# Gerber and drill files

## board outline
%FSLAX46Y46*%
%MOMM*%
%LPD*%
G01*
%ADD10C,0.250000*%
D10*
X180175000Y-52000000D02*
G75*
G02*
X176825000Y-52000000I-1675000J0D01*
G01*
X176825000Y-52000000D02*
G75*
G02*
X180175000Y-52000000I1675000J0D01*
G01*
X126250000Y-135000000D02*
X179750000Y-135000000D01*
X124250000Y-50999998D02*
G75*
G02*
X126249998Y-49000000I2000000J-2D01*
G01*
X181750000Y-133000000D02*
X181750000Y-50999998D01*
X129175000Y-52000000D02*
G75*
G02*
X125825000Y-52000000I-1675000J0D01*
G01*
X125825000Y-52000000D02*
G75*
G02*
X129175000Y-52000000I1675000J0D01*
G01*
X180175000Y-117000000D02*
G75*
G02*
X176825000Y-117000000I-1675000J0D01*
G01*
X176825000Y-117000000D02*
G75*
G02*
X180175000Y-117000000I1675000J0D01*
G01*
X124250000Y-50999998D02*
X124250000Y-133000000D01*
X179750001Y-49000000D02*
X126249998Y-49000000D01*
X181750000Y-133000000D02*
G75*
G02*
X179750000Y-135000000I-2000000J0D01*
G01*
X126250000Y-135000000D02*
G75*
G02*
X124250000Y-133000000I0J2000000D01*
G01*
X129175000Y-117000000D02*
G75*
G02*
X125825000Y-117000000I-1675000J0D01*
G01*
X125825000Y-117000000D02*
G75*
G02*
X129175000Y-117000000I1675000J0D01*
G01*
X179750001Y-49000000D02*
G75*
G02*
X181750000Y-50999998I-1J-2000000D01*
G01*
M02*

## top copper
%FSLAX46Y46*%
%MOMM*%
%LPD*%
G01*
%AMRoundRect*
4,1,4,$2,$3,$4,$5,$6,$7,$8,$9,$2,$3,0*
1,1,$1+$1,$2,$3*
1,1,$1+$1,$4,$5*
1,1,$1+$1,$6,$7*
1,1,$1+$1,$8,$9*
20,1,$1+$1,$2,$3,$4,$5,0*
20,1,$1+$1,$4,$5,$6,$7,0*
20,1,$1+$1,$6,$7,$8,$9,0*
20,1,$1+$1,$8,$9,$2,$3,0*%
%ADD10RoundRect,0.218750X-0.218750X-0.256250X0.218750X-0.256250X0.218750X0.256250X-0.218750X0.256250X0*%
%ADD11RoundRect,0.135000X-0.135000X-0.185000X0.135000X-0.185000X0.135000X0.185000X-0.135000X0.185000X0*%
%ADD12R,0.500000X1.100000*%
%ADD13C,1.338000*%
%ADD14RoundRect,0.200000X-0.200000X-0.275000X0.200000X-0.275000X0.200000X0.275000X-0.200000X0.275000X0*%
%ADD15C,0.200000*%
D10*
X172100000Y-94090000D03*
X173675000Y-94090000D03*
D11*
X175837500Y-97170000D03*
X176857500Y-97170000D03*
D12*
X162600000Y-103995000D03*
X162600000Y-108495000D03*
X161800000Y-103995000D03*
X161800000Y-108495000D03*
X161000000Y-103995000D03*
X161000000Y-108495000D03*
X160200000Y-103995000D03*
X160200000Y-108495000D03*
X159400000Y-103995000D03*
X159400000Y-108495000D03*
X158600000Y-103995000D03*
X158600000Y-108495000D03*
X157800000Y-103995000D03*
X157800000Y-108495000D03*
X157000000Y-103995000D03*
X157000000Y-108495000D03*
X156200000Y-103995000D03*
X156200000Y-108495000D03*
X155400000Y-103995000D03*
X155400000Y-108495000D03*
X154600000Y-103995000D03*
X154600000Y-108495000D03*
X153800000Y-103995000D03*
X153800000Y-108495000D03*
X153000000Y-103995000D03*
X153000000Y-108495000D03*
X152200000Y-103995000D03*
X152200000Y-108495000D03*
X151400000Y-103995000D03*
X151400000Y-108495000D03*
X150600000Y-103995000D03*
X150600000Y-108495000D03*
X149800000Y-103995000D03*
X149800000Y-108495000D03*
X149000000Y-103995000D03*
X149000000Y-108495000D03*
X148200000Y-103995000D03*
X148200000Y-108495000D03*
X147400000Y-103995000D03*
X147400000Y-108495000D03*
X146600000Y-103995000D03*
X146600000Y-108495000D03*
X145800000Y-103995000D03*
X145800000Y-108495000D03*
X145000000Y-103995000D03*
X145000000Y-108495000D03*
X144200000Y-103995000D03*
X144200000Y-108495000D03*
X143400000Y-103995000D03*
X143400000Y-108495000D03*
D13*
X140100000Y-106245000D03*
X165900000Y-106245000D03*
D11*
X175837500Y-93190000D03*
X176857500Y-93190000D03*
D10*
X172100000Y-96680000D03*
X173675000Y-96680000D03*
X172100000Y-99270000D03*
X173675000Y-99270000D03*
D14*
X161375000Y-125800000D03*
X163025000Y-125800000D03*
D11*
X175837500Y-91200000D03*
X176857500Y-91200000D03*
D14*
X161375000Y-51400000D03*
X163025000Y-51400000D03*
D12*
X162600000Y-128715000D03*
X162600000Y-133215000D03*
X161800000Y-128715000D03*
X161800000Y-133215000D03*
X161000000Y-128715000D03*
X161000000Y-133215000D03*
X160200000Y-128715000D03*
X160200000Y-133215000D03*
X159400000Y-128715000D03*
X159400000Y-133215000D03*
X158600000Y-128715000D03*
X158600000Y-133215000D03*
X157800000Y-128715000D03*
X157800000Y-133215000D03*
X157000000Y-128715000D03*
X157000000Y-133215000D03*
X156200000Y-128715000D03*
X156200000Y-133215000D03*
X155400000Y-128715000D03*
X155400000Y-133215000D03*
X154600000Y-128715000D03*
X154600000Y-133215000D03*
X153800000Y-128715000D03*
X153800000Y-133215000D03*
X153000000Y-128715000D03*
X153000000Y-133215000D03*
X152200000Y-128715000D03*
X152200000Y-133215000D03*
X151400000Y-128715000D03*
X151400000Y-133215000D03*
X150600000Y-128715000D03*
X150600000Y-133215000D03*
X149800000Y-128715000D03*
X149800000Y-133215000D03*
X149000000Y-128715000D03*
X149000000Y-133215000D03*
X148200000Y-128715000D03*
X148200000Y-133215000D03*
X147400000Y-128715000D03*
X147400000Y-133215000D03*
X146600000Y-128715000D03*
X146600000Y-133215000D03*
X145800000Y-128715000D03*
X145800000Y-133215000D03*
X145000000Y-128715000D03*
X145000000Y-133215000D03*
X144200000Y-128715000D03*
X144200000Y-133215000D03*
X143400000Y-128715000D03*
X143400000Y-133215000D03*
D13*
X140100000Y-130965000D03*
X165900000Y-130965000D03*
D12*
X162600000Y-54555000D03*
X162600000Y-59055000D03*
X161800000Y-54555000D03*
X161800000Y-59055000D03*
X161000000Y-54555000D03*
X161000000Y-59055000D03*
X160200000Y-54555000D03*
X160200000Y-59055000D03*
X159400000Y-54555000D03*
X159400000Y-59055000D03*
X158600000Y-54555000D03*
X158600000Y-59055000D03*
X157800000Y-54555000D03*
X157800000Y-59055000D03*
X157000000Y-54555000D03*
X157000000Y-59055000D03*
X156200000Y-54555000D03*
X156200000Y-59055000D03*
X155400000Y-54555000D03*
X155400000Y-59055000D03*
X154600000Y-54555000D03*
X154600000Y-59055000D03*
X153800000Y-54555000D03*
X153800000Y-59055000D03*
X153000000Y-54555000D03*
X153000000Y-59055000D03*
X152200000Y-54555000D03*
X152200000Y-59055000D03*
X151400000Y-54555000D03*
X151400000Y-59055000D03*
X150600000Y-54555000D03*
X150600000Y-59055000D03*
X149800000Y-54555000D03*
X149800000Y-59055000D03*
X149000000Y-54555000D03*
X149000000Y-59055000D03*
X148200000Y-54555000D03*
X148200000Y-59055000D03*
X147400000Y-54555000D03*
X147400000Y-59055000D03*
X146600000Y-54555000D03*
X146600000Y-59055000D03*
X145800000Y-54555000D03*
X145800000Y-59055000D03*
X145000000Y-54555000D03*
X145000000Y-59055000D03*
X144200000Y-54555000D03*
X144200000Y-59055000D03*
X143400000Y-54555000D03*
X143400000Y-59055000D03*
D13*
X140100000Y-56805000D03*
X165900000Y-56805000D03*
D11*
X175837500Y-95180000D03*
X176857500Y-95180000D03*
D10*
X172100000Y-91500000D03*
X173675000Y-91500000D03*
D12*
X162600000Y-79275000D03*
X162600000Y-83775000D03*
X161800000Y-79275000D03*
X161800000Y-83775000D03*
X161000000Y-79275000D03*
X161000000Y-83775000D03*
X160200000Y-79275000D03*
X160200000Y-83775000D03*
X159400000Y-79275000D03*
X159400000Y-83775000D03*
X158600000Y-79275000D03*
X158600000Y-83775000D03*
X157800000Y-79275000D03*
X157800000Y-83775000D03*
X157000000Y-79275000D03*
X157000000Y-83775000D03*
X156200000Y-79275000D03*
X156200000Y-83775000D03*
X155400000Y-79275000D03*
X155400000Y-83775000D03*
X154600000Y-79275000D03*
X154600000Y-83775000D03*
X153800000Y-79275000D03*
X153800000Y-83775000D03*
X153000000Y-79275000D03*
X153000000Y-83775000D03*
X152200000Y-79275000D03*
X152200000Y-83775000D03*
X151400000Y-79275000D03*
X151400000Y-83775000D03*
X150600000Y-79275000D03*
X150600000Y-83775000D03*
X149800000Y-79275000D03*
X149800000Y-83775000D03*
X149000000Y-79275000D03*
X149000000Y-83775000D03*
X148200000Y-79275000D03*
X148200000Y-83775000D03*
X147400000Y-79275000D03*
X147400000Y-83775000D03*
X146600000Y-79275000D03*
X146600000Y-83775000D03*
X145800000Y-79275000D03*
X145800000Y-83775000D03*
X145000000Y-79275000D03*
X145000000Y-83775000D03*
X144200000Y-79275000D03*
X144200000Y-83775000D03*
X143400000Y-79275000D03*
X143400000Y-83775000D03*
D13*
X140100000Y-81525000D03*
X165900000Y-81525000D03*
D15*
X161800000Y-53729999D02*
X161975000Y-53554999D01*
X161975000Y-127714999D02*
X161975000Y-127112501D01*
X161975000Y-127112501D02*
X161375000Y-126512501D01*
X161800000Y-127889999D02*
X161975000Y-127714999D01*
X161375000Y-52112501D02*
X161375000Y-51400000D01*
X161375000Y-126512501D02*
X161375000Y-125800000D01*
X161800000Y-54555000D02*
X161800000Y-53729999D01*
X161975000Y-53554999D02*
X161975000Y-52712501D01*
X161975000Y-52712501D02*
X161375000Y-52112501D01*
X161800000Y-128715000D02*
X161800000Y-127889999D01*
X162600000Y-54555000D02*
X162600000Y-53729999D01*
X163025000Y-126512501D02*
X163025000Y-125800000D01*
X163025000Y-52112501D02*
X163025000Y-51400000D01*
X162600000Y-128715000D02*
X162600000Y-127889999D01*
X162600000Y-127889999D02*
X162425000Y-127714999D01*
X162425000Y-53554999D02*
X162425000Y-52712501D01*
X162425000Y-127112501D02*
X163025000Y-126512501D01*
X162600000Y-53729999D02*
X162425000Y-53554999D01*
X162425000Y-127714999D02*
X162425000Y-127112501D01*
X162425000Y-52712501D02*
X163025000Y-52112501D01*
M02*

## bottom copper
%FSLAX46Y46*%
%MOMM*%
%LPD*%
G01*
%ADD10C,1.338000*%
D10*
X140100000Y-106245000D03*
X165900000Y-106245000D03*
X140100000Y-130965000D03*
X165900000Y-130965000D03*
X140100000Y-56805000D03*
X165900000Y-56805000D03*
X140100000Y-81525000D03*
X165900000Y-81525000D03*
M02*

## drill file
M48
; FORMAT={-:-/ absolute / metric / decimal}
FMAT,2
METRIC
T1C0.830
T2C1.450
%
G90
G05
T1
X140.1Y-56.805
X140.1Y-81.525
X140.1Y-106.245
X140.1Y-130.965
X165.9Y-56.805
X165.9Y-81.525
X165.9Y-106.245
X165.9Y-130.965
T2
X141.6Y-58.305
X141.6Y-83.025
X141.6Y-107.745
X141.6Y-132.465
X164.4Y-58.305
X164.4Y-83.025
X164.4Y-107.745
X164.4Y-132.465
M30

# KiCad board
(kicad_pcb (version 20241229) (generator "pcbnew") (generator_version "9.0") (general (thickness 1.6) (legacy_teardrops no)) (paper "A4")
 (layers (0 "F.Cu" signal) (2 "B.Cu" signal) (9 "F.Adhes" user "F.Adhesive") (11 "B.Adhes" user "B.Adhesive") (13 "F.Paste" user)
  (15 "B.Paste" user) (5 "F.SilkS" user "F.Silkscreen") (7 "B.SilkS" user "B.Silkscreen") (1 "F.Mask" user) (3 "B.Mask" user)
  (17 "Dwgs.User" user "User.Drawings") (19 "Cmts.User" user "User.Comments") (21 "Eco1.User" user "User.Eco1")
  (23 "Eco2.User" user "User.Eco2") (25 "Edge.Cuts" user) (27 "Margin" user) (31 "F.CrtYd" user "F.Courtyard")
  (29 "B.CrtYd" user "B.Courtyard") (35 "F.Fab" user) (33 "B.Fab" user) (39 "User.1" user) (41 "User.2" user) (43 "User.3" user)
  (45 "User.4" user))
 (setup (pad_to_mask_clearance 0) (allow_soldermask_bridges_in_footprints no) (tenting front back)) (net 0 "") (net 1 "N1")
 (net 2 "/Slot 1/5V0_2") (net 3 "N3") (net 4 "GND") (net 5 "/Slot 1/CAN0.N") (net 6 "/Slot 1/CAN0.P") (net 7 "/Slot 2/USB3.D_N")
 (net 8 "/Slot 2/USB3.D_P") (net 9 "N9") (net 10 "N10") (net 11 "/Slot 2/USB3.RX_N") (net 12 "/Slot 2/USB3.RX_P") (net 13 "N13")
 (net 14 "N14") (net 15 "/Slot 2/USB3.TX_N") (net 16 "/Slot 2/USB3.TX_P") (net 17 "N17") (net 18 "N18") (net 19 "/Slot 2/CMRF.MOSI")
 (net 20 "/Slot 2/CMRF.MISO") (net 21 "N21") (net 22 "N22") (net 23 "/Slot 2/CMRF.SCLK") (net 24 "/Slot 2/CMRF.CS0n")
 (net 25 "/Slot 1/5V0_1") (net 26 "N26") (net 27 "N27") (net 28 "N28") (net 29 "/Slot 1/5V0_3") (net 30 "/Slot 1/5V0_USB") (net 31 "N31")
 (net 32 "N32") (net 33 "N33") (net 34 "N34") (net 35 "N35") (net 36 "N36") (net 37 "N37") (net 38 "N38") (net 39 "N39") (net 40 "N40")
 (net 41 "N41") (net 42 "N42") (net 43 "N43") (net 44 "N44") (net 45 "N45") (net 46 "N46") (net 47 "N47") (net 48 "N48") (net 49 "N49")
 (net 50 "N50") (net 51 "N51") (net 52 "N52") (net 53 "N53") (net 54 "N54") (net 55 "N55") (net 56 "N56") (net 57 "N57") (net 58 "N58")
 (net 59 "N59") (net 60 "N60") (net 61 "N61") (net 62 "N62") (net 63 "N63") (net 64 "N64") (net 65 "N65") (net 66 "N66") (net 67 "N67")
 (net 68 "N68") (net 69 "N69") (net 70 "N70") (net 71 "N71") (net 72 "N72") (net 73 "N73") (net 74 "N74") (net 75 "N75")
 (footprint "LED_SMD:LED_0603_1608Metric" (layer "F.Cu") (at 172.8875 94.09)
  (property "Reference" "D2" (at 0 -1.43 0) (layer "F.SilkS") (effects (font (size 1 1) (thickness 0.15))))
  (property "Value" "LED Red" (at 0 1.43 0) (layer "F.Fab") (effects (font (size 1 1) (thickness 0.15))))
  (pad "1" smd roundrect (at -0.7875 0) (size 0.875 0.95) (layers "F.Cu" "F.Mask" "F.Paste") (roundrect_rratio 0.25) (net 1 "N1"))
  (pad "2" smd roundrect (at 0.7875 0) (size 0.875 0.95) (layers "F.Cu" "F.Mask" "F.Paste") (roundrect_rratio 0.25) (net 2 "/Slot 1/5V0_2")))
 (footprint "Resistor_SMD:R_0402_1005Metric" (layer "F.Cu") (at 176.3475 97.17)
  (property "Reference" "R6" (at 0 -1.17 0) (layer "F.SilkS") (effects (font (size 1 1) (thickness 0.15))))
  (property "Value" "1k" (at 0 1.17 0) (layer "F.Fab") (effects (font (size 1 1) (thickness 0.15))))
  (pad "1" smd roundrect (at -0.51 0) (size 0.54 0.64) (layers "F.Cu" "F.Mask" "F.Paste") (roundrect_rratio 0.25) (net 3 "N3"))
  (pad "2" smd roundrect (at 0.51 0) (size 0.54 0.64) (layers "F.Cu" "F.Mask" "F.Paste") (roundrect_rratio 0.25) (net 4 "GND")))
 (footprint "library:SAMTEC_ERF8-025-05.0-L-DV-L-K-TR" (layer "F.Cu") (at 153 106.245)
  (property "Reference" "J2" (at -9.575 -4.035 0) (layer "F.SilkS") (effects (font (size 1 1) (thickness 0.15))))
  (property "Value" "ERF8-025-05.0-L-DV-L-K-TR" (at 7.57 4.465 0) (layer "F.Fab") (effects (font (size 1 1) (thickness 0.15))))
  (pad "" np_thru_hole circle (at -11.4 1.5) (size 1.45 1.45) (drill 1.45) (layers "*.Cu" "*.Mask"))
  (pad "" np_thru_hole circle (at 11.4 1.5) (size 1.45 1.45) (drill 1.45) (layers "*.Cu" "*.Mask"))
  (pad "01" smd rect (at 9.6 -2.25) (size 0.5 1.1) (layers "F.Cu" "F.Mask" "F.Paste") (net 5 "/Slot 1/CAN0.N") (solder_mask_margin 0.102))
  (pad "02" smd rect (at 9.6 2.25) (size 0.5 1.1) (layers "F.Cu" "F.Mask" "F.Paste") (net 4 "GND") (solder_mask_margin 0.102))
  (pad "03" smd rect (at 8.8 -2.25) (size 0.5 1.1) (layers "F.Cu" "F.Mask" "F.Paste") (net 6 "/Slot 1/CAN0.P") (solder_mask_margin 0.102))
  (pad "04" smd rect (at 8.8 2.25) (size 0.5 1.1) (layers "F.Cu" "F.Mask" "F.Paste") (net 4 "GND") (solder_mask_margin 0.102))
  (pad "05" smd rect (at 8 -2.25) (size 0.5 1.1) (layers "F.Cu" "F.Mask" "F.Paste") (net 4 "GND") (solder_mask_margin 0.102))
  (pad "06" smd rect (at 8 2.25) (size 0.5 1.1) (layers "F.Cu" "F.Mask" "F.Paste") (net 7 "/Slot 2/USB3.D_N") (solder_mask_margin 0.102))
  (pad "07" smd rect (at 7.2 -2.25) (size 0.5 1.1) (layers "F.Cu" "F.Mask" "F.Paste") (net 4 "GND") (solder_mask_margin 0.102))
  (pad "08" smd rect (at 7.2 2.25) (size 0.5 1.1) (layers "F.Cu" "F.Mask" "F.Paste") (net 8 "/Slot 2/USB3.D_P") (solder_mask_margin 0.102))
  (pad "09" smd rect (at 6.4 -2.25) (size 0.5 1.1) (layers "F.Cu" "F.Mask" "F.Paste") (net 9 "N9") (solder_mask_margin 0.102))
  (pad "10" smd rect (at 6.4 2.25) (size 0.5 1.1) (layers "F.Cu" "F.Mask" "F.Paste") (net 4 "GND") (solder_mask_margin 0.102))
  (pad "11" smd rect (at 5.6 -2.25) (size 0.5 1.1) (layers "F.Cu" "F.Mask" "F.Paste") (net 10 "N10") (solder_mask_margin 0.102))
  (pad "12" smd rect (at 5.6 2.25) (size 0.5 1.1) (layers "F.Cu" "F.Mask" "F.Paste") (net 4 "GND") (solder_mask_margin 0.102))
  (pad "13" smd rect (at 4.8 -2.25) (size 0.5 1.1) (layers "F.Cu" "F.Mask" "F.Paste") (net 4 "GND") (solder_mask_margin 0.102))
  (pad "14" smd rect (at 4.8 2.25) (size 0.5 1.1) (layers "F.Cu" "F.Mask" "F.Paste") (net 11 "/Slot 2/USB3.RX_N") (solder_mask_margin 0.102))
  (pad "15" smd rect (at 4 -2.25) (size 0.5 1.1) (layers "F.Cu" "F.Mask" "F.Paste") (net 4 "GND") (solder_mask_margin 0.102))
  (pad "16" smd rect (at 4 2.25) (size 0.5 1.1) (layers "F.Cu" "F.Mask" "F.Paste") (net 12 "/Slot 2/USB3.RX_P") (solder_mask_margin 0.102))
  (pad "17" smd rect (at 3.2 -2.25) (size 0.5 1.1) (layers "F.Cu" "F.Mask" "F.Paste") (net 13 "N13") (solder_mask_margin 0.102))
  (pad "18" smd rect (at 3.2 2.25) (size 0.5 1.1) (layers "F.Cu" "F.Mask" "F.Paste") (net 4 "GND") (solder_mask_margin 0.102))
  (pad "19" smd rect (at 2.4 -2.25) (size 0.5 1.1) (layers "F.Cu" "F.Mask" "F.Paste") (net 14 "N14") (solder_mask_margin 0.102))
  (pad "20" smd rect (at 2.4 2.25) (size 0.5 1.1) (layers "F.Cu" "F.Mask" "F.Paste") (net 4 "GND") (solder_mask_margin 0.102))
  (pad "21" smd rect (at 1.6 -2.25) (size 0.5 1.1) (layers "F.Cu" "F.Mask" "F.Paste") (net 4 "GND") (solder_mask_margin 0.102))
  (pad "22" smd rect (at 1.6 2.25) (size 0.5 1.1) (layers "F.Cu" "F.Mask" "F.Paste") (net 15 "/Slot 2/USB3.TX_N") (solder_mask_margin 0.102))
  (pad "23" smd rect (at 0.8 -2.25) (size 0.5 1.1) (layers "F.Cu" "F.Mask" "F.Paste") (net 4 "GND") (solder_mask_margin 0.102))
  (pad "24" smd rect (at 0.8 2.25) (size 0.5 1.1) (layers "F.Cu" "F.Mask" "F.Paste") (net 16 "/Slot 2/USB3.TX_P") (solder_mask_margin 0.102))
  (pad "25" smd rect (at 0 -2.25) (size 0.5 1.1) (layers "F.Cu" "F.Mask" "F.Paste") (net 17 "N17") (solder_mask_margin 0.102))
  (pad "26" smd rect (at 0 2.25) (size 0.5 1.1) (layers "F.Cu" "F.Mask" "F.Paste") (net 4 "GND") (solder_mask_margin 0.102))
  (pad "27" smd rect (at -0.8 -2.25) (size 0.5 1.1) (layers "F.Cu" "F.Mask" "F.Paste") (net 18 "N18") (solder_mask_margin 0.102))
  (pad "28" smd rect (at -0.8 2.25) (size 0.5 1.1) (layers "F.Cu" "F.Mask" "F.Paste") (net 4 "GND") (solder_mask_margin 0.102))
  (pad "29" smd rect (at -1.6 -2.25) (size 0.5 1.1) (layers "F.Cu" "F.Mask" "F.Paste") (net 4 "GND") (solder_mask_margin 0.102))
  (pad "30" smd rect (at -1.6 2.25) (size 0.5 1.1) (layers "F.Cu" "F.Mask" "F.Paste") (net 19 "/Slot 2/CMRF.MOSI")
   (solder_mask_margin 0.102))
  (pad "31" smd rect (at -2.4 -2.25) (size 0.5 1.1) (layers "F.Cu" "F.Mask" "F.Paste") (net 4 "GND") (solder_mask_margin 0.102))
  (pad "32" smd rect (at -2.4 2.25) (size 0.5 1.1) (layers "F.Cu" "F.Mask" "F.Paste") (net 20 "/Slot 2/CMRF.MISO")
   (solder_mask_margin 0.102))
  (pad "33" smd rect (at -3.2 -2.25) (size 0.5 1.1) (layers "F.Cu" "F.Mask" "F.Paste") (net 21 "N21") (solder_mask_margin 0.102))
  (pad "34" smd rect (at -3.2 2.25) (size 0.5 1.1) (layers "F.Cu" "F.Mask" "F.Paste") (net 4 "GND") (solder_mask_margin 0.102))
  (pad "35" smd rect (at -4 -2.25) (size 0.5 1.1) (layers "F.Cu" "F.Mask" "F.Paste") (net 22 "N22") (solder_mask_margin 0.102))
  (pad "36" smd rect (at -4 2.25) (size 0.5 1.1) (layers "F.Cu" "F.Mask" "F.Paste") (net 4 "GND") (solder_mask_margin 0.102))
  (pad "37" smd rect (at -4.8 -2.25) (size 0.5 1.1) (layers "F.Cu" "F.Mask" "F.Paste") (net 4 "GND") (solder_mask_margin 0.102))
  (pad "38" smd rect (at -4.8 2.25) (size 0.5 1.1) (layers "F.Cu" "F.Mask" "F.Paste") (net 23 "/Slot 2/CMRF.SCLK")
   (solder_mask_margin 0.102))
  (pad "39" smd rect (at -5.6 -2.25) (size 0.5 1.1) (layers "F.Cu" "F.Mask" "F.Paste") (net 4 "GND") (solder_mask_margin 0.102))
  (pad "40" smd rect (at -5.6 2.25) (size 0.5 1.1) (layers "F.Cu" "F.Mask" "F.Paste") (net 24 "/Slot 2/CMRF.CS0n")
   (solder_mask_margin 0.102))
  (pad "41" smd rect (at -6.4 -2.25) (size 0.5 1.1) (layers "F.Cu" "F.Mask" "F.Paste") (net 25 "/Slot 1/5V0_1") (solder_mask_margin 0.102))
  (pad "42" smd rect (at -6.4 2.25) (size 0.5 1.1) (layers "F.Cu" "F.Mask" "F.Paste") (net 4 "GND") (solder_mask_margin 0.102))
  (pad "43" smd rect (at -7.2 -2.25) (size 0.5 1.1) (layers "F.Cu" "F.Mask" "F.Paste") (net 25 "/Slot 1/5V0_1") (solder_mask_margin 0.102))
  (pad "44" smd rect (at -7.2 2.25) (size 0.5 1.1) (layers "F.Cu" "F.Mask" "F.Paste") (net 4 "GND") (solder_mask_margin 0.102))
  (pad "45" smd rect (at -8 -2.25) (size 0.5 1.1) (layers "F.Cu" "F.Mask" "F.Paste") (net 25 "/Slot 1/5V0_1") (solder_mask_margin 0.102))
  (pad "46" smd rect (at -8 2.25) (size 0.5 1.1) (layers "F.Cu" "F.Mask" "F.Paste") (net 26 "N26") (solder_mask_margin 0.102))
  (pad "47" smd rect (at -8.8 -2.25) (size 0.5 1.1) (layers "F.Cu" "F.Mask" "F.Paste") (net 25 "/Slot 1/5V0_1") (solder_mask_margin 0.102))
  (pad "48" smd rect (at -8.8 2.25) (size 0.5 1.1) (layers "F.Cu" "F.Mask" "F.Paste") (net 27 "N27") (solder_mask_margin 0.102))
  (pad "49" smd rect (at -9.6 -2.25) (size 0.5 1.1) (layers "F.Cu" "F.Mask" "F.Paste") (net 25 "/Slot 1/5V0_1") (solder_mask_margin 0.102))
  (pad "50" smd rect (at -9.6 2.25) (size 0.5 1.1) (layers "F.Cu" "F.Mask" "F.Paste") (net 4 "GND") (solder_mask_margin 0.102))
  (pad "S1" thru_hole circle (at -12.9 0) (size 1.338 1.338) (drill 0.83) (layers "*.Cu" "*.Mask") (remove_unused_layers no)
   (solder_mask_margin 0.102))
  (pad "S2" thru_hole circle (at 12.9 0) (size 1.338 1.338) (drill 0.83) (layers "*.Cu" "*.Mask") (remove_unused_layers no)
   (solder_mask_margin 0.102)))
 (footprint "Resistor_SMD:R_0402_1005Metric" (layer "F.Cu") (at 176.3475 93.19)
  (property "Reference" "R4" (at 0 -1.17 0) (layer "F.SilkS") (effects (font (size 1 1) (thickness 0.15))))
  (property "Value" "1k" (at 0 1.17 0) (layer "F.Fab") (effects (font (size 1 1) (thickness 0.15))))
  (pad "1" smd roundrect (at -0.51 0) (size 0.54 0.64) (layers "F.Cu" "F.Mask" "F.Paste") (roundrect_rratio 0.25) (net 1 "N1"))
  (pad "2" smd roundrect (at 0.51 0) (size 0.54 0.64) (layers "F.Cu" "F.Mask" "F.Paste") (roundrect_rratio 0.25) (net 4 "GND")))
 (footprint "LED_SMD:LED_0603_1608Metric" (layer "F.Cu") (at 172.8875 96.68)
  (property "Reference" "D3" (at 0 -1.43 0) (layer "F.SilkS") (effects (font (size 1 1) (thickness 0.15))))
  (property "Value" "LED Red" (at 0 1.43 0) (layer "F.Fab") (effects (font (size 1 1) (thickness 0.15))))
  (pad "1" smd roundrect (at -0.7875 0) (size 0.875 0.95) (layers "F.Cu" "F.Mask" "F.Paste") (roundrect_rratio 0.25) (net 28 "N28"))
  (pad "2" smd roundrect (at 0.7875 0) (size 0.875 0.95) (layers "F.Cu" "F.Mask" "F.Paste") (roundrect_rratio 0.25) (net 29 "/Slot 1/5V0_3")))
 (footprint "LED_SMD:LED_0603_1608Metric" (layer "F.Cu") (at 172.8875 99.27)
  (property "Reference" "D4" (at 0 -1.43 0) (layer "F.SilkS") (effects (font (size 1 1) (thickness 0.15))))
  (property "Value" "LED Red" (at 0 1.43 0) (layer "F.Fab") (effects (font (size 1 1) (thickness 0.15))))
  (pad "1" smd roundrect (at -0.7875 0) (size 0.875 0.95) (layers "F.Cu" "F.Mask" "F.Paste") (roundrect_rratio 0.25) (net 3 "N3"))
  (pad "2" smd roundrect (at 0.7875 0) (size 0.875 0.95) (layers "F.Cu" "F.Mask" "F.Paste") (roundrect_rratio 0.25)
   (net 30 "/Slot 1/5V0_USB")))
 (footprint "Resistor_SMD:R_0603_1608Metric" (layer "F.Cu") (at 162.2 125.8)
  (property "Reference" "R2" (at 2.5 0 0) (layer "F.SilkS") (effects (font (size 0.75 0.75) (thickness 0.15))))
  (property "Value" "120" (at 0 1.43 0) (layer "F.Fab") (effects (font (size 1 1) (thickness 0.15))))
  (pad "1" smd roundrect (at -0.825 0) (size 0.8 0.95) (layers "F.Cu" "F.Mask" "F.Paste") (roundrect_rratio 0.25) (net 6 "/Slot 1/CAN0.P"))
  (pad "2" smd roundrect (at 0.825 0) (size 0.8 0.95) (layers "F.Cu" "F.Mask" "F.Paste") (roundrect_rratio 0.25) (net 5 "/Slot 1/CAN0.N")))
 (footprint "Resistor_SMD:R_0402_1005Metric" (layer "F.Cu") (at 176.3475 91.2)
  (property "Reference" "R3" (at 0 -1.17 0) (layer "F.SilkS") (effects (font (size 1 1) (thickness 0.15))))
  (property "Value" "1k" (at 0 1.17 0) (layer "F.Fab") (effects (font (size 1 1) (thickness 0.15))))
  (pad "1" smd roundrect (at -0.51 0) (size 0.54 0.64) (layers "F.Cu" "F.Mask" "F.Paste") (roundrect_rratio 0.25) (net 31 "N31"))
  (pad "2" smd roundrect (at 0.51 0) (size 0.54 0.64) (layers "F.Cu" "F.Mask" "F.Paste") (roundrect_rratio 0.25) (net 4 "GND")))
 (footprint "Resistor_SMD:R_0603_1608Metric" (layer "F.Cu") (at 162.2 51.4)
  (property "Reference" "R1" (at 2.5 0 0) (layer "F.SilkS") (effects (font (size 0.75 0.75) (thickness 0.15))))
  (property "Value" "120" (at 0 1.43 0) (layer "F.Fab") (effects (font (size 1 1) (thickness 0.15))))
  (pad "1" smd roundrect (at -0.825 0) (size 0.8 0.95) (layers "F.Cu" "F.Mask" "F.Paste") (roundrect_rratio 0.25) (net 6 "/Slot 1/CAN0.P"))
  (pad "2" smd roundrect (at 0.825 0) (size 0.8 0.95) (layers "F.Cu" "F.Mask" "F.Paste") (roundrect_rratio 0.25) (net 5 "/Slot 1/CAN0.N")))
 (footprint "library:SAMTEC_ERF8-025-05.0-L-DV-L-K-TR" (layer "F.Cu") (at 153 130.965)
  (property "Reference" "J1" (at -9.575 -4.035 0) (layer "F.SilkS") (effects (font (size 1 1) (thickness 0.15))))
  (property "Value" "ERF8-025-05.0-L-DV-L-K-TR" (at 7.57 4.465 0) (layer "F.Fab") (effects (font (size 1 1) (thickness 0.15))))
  (pad "" np_thru_hole circle (at -11.4 1.5) (size 1.45 1.45) (drill 1.45) (layers "*.Cu" "*.Mask"))
  (pad "" np_thru_hole circle (at 11.4 1.5) (size 1.45 1.45) (drill 1.45) (layers "*.Cu" "*.Mask"))
  (pad "01" smd rect (at 9.6 -2.25) (size 0.5 1.1) (layers "F.Cu" "F.Mask" "F.Paste") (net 5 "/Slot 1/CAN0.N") (solder_mask_margin 0.102))
  (pad "02" smd rect (at 9.6 2.25) (size 0.5 1.1) (layers "F.Cu" "F.Mask" "F.Paste") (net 4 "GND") (solder_mask_margin 0.102))
  (pad "03" smd rect (at 8.8 -2.25) (size 0.5 1.1) (layers "F.Cu" "F.Mask" "F.Paste") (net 6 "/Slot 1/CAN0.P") (solder_mask_margin 0.102))
  (pad "04" smd rect (at 8.8 2.25) (size 0.5 1.1) (layers "F.Cu" "F.Mask" "F.Paste") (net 4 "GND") (solder_mask_margin 0.102))
  (pad "05" smd rect (at 8 -2.25) (size 0.5 1.1) (layers "F.Cu" "F.Mask" "F.Paste") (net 4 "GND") (solder_mask_margin 0.102))
  (pad "06" smd rect (at 8 2.25) (size 0.5 1.1) (layers "F.Cu" "F.Mask" "F.Paste") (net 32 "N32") (solder_mask_margin 0.102))
  (pad "07" smd rect (at 7.2 -2.25) (size 0.5 1.1) (layers "F.Cu" "F.Mask" "F.Paste") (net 4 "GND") (solder_mask_margin 0.102))
  (pad "08" smd rect (at 7.2 2.25) (size 0.5 1.1) (layers "F.Cu" "F.Mask" "F.Paste") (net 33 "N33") (solder_mask_margin 0.102))
  (pad "09" smd rect (at 6.4 -2.25) (size 0.5 1.1) (layers "F.Cu" "F.Mask" "F.Paste") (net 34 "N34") (solder_mask_margin 0.102))
  (pad "10" smd rect (at 6.4 2.25) (size 0.5 1.1) (layers "F.Cu" "F.Mask" "F.Paste") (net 4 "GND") (solder_mask_margin 0.102))
  (pad "11" smd rect (at 5.6 -2.25) (size 0.5 1.1) (layers "F.Cu" "F.Mask" "F.Paste") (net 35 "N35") (solder_mask_margin 0.102))
  (pad "12" smd rect (at 5.6 2.25) (size 0.5 1.1) (layers "F.Cu" "F.Mask" "F.Paste") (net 4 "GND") (solder_mask_margin 0.102))
  (pad "13" smd rect (at 4.8 -2.25) (size 0.5 1.1) (layers "F.Cu" "F.Mask" "F.Paste") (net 4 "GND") (solder_mask_margin 0.102))
  (pad "14" smd rect (at 4.8 2.25) (size 0.5 1.1) (layers "F.Cu" "F.Mask" "F.Paste") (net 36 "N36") (solder_mask_margin 0.102))
  (pad "15" smd rect (at 4 -2.25) (size 0.5 1.1) (layers "F.Cu" "F.Mask" "F.Paste") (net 4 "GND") (solder_mask_margin 0.102))
  (pad "16" smd rect (at 4 2.25) (size 0.5 1.1) (layers "F.Cu" "F.Mask" "F.Paste") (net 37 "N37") (solder_mask_margin 0.102))
  (pad "17" smd rect (at 3.2 -2.25) (size 0.5 1.1) (layers "F.Cu" "F.Mask" "F.Paste") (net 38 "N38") (solder_mask_margin 0.102))
  (pad "18" smd rect (at 3.2 2.25) (size 0.5 1.1) (layers "F.Cu" "F.Mask" "F.Paste") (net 4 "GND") (solder_mask_margin 0.102))
  (pad "19" smd rect (at 2.4 -2.25) (size 0.5 1.1) (layers "F.Cu" "F.Mask" "F.Paste") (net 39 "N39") (solder_mask_margin 0.102))
  (pad "20" smd rect (at 2.4 2.25) (size 0.5 1.1) (layers "F.Cu" "F.Mask" "F.Paste") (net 4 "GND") (solder_mask_margin 0.102))
  (pad "21" smd rect (at 1.6 -2.25) (size 0.5 1.1) (layers "F.Cu" "F.Mask" "F.Paste") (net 4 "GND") (solder_mask_margin 0.102))
  (pad "22" smd rect (at 1.6 2.25) (size 0.5 1.1) (layers "F.Cu" "F.Mask" "F.Paste") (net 4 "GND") (solder_mask_margin 0.102))
  (pad "23" smd rect (at 0.8 -2.25) (size 0.5 1.1) (layers "F.Cu" "F.Mask" "F.Paste") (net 4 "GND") (solder_mask_margin 0.102))
  (pad "24" smd rect (at 0.8 2.25) (size 0.5 1.1) (layers "F.Cu" "F.Mask" "F.Paste") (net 4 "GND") (solder_mask_margin 0.102))
  (pad "25" smd rect (at 0 -2.25) (size 0.5 1.1) (layers "F.Cu" "F.Mask" "F.Paste") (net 4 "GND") (solder_mask_margin 0.102))
  (pad "26" smd rect (at 0 2.25) (size 0.5 1.1) (layers "F.Cu" "F.Mask" "F.Paste") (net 4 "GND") (solder_mask_margin 0.102))
  (pad "27" smd rect (at -0.8 -2.25) (size 0.5 1.1) (layers "F.Cu" "F.Mask" "F.Paste") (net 4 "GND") (solder_mask_margin 0.102))
  (pad "28" smd rect (at -0.8 2.25) (size 0.5 1.1) (layers "F.Cu" "F.Mask" "F.Paste") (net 4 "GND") (solder_mask_margin 0.102))
  (pad "29" smd rect (at -1.6 -2.25) (size 0.5 1.1) (layers "F.Cu" "F.Mask" "F.Paste") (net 4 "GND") (solder_mask_margin 0.102))
  (pad "30" smd rect (at -1.6 2.25) (size 0.5 1.1) (layers "F.Cu" "F.Mask" "F.Paste") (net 4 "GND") (solder_mask_margin 0.102))
  (pad "31" smd rect (at -2.4 -2.25) (size 0.5 1.1) (layers "F.Cu" "F.Mask" "F.Paste") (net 29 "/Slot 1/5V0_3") (solder_mask_margin 0.102))
  (pad "32" smd rect (at -2.4 2.25) (size 0.5 1.1) (layers "F.Cu" "F.Mask" "F.Paste") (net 30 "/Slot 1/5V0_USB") (solder_mask_margin 0.102))
  (pad "33" smd rect (at -3.2 -2.25) (size 0.5 1.1) (layers "F.Cu" "F.Mask" "F.Paste") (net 29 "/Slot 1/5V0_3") (solder_mask_margin 0.102))
  (pad "34" smd rect (at -3.2 2.25) (size 0.5 1.1) (layers "F.Cu" "F.Mask" "F.Paste") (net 30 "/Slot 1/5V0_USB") (solder_mask_margin 0.102))
  (pad "35" smd rect (at -4 -2.25) (size 0.5 1.1) (layers "F.Cu" "F.Mask" "F.Paste") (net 29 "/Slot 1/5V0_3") (solder_mask_margin 0.102))
  (pad "36" smd rect (at -4 2.25) (size 0.5 1.1) (layers "F.Cu" "F.Mask" "F.Paste") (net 30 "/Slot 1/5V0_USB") (solder_mask_margin 0.102))
  (pad "37" smd rect (at -4.8 -2.25) (size 0.5 1.1) (layers "F.Cu" "F.Mask" "F.Paste") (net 29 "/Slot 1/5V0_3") (solder_mask_margin 0.102))
  (pad "38" smd rect (at -4.8 2.25) (size 0.5 1.1) (layers "F.Cu" "F.Mask" "F.Paste") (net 30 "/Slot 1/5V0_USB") (solder_mask_margin 0.102))
  (pad "39" smd rect (at -5.6 -2.25) (size 0.5 1.1) (layers "F.Cu" "F.Mask" "F.Paste") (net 29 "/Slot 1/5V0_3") (solder_mask_margin 0.102))
  (pad "40" smd rect (at -5.6 2.25) (size 0.5 1.1) (layers "F.Cu" "F.Mask" "F.Paste") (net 30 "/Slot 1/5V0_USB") (solder_mask_margin 0.102))
  (pad "41" smd rect (at -6.4 -2.25) (size 0.5 1.1) (layers "F.Cu" "F.Mask" "F.Paste") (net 25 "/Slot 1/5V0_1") (solder_mask_margin 0.102))
  (pad "42" smd rect (at -6.4 2.25) (size 0.5 1.1) (layers "F.Cu" "F.Mask" "F.Paste") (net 2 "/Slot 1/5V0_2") (solder_mask_margin 0.102))
  (pad "43" smd rect (at -7.2 -2.25) (size 0.5 1.1) (layers "F.Cu" "F.Mask" "F.Paste") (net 25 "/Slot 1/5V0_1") (solder_mask_margin 0.102))
  (pad "44" smd rect (at -7.2 2.25) (size 0.5 1.1) (layers "F.Cu" "F.Mask" "F.Paste") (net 2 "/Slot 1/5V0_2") (solder_mask_margin 0.102))
  (pad "45" smd rect (at -8 -2.25) (size 0.5 1.1) (layers "F.Cu" "F.Mask" "F.Paste") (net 25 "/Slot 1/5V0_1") (solder_mask_margin 0.102))
  (pad "46" smd rect (at -8 2.25) (size 0.5 1.1) (layers "F.Cu" "F.Mask" "F.Paste") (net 2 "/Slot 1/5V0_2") (solder_mask_margin 0.102))
  (pad "47" smd rect (at -8.8 -2.25) (size 0.5 1.1) (layers "F.Cu" "F.Mask" "F.Paste") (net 25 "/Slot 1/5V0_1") (solder_mask_margin 0.102))
  (pad "48" smd rect (at -8.8 2.25) (size 0.5 1.1) (layers "F.Cu" "F.Mask" "F.Paste") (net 2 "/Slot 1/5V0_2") (solder_mask_margin 0.102))
  (pad "49" smd rect (at -9.6 -2.25) (size 0.5 1.1) (layers "F.Cu" "F.Mask" "F.Paste") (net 25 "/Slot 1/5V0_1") (solder_mask_margin 0.102))
  (pad "50" smd rect (at -9.6 2.25) (size 0.5 1.1) (layers "F.Cu" "F.Mask" "F.Paste") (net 2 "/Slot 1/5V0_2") (solder_mask_margin 0.102))
  (pad "S1" thru_hole circle (at -12.9 0) (size 1.338 1.338) (drill 0.83) (layers "*.Cu" "*.Mask") (remove_unused_layers no)
   (solder_mask_margin 0.102))
  (pad "S2" thru_hole circle (at 12.9 0) (size 1.338 1.338) (drill 0.83) (layers "*.Cu" "*.Mask") (remove_unused_layers no)
   (solder_mask_margin 0.102)))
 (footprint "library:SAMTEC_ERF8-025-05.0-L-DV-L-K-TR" (layer "F.Cu") (at 153 56.805)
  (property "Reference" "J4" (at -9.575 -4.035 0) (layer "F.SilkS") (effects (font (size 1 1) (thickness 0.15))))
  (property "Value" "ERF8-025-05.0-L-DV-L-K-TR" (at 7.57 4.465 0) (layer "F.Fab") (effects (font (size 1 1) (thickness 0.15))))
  (pad "" np_thru_hole circle (at -11.4 1.5) (size 1.45 1.45) (drill 1.45) (layers "*.Cu" "*.Mask"))
  (pad "" np_thru_hole circle (at 11.4 1.5) (size 1.45 1.45) (drill 1.45) (layers "*.Cu" "*.Mask"))
  (pad "01" smd rect (at 9.6 -2.25) (size 0.5 1.1) (layers "F.Cu" "F.Mask" "F.Paste") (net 5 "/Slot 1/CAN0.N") (solder_mask_margin 0.102))
  (pad "02" smd rect (at 9.6 2.25) (size 0.5 1.1) (layers "F.Cu" "F.Mask" "F.Paste") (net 4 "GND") (solder_mask_margin 0.102))
  (pad "03" smd rect (at 8.8 -2.25) (size 0.5 1.1) (layers "F.Cu" "F.Mask" "F.Paste") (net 6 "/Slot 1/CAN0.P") (solder_mask_margin 0.102))
  (pad "04" smd rect (at 8.8 2.25) (size 0.5 1.1) (layers "F.Cu" "F.Mask" "F.Paste") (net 4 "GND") (solder_mask_margin 0.102))
  (pad "05" smd rect (at 8 -2.25) (size 0.5 1.1) (layers "F.Cu" "F.Mask" "F.Paste") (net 4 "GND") (solder_mask_margin 0.102))
  (pad "06" smd rect (at 8 2.25) (size 0.5 1.1) (layers "F.Cu" "F.Mask" "F.Paste") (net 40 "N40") (solder_mask_margin 0.102))
  (pad "07" smd rect (at 7.2 -2.25) (size 0.5 1.1) (layers "F.Cu" "F.Mask" "F.Paste") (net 4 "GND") (solder_mask_margin 0.102))
  (pad "08" smd rect (at 7.2 2.25) (size 0.5 1.1) (layers "F.Cu" "F.Mask" "F.Paste") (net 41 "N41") (solder_mask_margin 0.102))
  (pad "09" smd rect (at 6.4 -2.25) (size 0.5 1.1) (layers "F.Cu" "F.Mask" "F.Paste") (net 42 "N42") (solder_mask_margin 0.102))
  (pad "10" smd rect (at 6.4 2.25) (size 0.5 1.1) (layers "F.Cu" "F.Mask" "F.Paste") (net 4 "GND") (solder_mask_margin 0.102))
  (pad "11" smd rect (at 5.6 -2.25) (size 0.5 1.1) (layers "F.Cu" "F.Mask" "F.Paste") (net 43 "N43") (solder_mask_margin 0.102))
  (pad "12" smd rect (at 5.6 2.25) (size 0.5 1.1) (layers "F.Cu" "F.Mask" "F.Paste") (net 4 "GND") (solder_mask_margin 0.102))
  (pad "13" smd rect (at 4.8 -2.25) (size 0.5 1.1) (layers "F.Cu" "F.Mask" "F.Paste") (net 4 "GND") (solder_mask_margin 0.102))
  (pad "14" smd rect (at 4.8 2.25) (size 0.5 1.1) (layers "F.Cu" "F.Mask" "F.Paste") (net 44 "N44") (solder_mask_margin 0.102))
  (pad "15" smd rect (at 4 -2.25) (size 0.5 1.1) (layers "F.Cu" "F.Mask" "F.Paste") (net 4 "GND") (solder_mask_margin 0.102))
  (pad "16" smd rect (at 4 2.25) (size 0.5 1.1) (layers "F.Cu" "F.Mask" "F.Paste") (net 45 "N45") (solder_mask_margin 0.102))
  (pad "17" smd rect (at 3.2 -2.25) (size 0.5 1.1) (layers "F.Cu" "F.Mask" "F.Paste") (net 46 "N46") (solder_mask_margin 0.102))
  (pad "18" smd rect (at 3.2 2.25) (size 0.5 1.1) (layers "F.Cu" "F.Mask" "F.Paste") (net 4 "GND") (solder_mask_margin 0.102))
  (pad "19" smd rect (at 2.4 -2.25) (size 0.5 1.1) (layers "F.Cu" "F.Mask" "F.Paste") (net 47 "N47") (solder_mask_margin 0.102))
  (pad "20" smd rect (at 2.4 2.25) (size 0.5 1.1) (layers "F.Cu" "F.Mask" "F.Paste") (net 4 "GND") (solder_mask_margin 0.102))
  (pad "21" smd rect (at 1.6 -2.25) (size 0.5 1.1) (layers "F.Cu" "F.Mask" "F.Paste") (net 4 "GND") (solder_mask_margin 0.102))
  (pad "22" smd rect (at 1.6 2.25) (size 0.5 1.1) (layers "F.Cu" "F.Mask" "F.Paste") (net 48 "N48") (solder_mask_margin 0.102))
  (pad "23" smd rect (at 0.8 -2.25) (size 0.5 1.1) (layers "F.Cu" "F.Mask" "F.Paste") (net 4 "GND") (solder_mask_margin 0.102))
  (pad "24" smd rect (at 0.8 2.25) (size 0.5 1.1) (layers "F.Cu" "F.Mask" "F.Paste") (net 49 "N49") (solder_mask_margin 0.102))
  (pad "25" smd rect (at 0 -2.25) (size 0.5 1.1) (layers "F.Cu" "F.Mask" "F.Paste") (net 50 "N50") (solder_mask_margin 0.102))
  (pad "26" smd rect (at 0 2.25) (size 0.5 1.1) (layers "F.Cu" "F.Mask" "F.Paste") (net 4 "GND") (solder_mask_margin 0.102))
  (pad "27" smd rect (at -0.8 -2.25) (size 0.5 1.1) (layers "F.Cu" "F.Mask" "F.Paste") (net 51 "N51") (solder_mask_margin 0.102))
  (pad "28" smd rect (at -0.8 2.25) (size 0.5 1.1) (layers "F.Cu" "F.Mask" "F.Paste") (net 4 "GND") (solder_mask_margin 0.102))
  (pad "29" smd rect (at -1.6 -2.25) (size 0.5 1.1) (layers "F.Cu" "F.Mask" "F.Paste") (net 4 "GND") (solder_mask_margin 0.102))
  (pad "30" smd rect (at -1.6 2.25) (size 0.5 1.1) (layers "F.Cu" "F.Mask" "F.Paste") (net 19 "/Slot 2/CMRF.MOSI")
   (solder_mask_margin 0.102))
  (pad "31" smd rect (at -2.4 -2.25) (size 0.5 1.1) (layers "F.Cu" "F.Mask" "F.Paste") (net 4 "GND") (solder_mask_margin 0.102))
  (pad "32" smd rect (at -2.4 2.25) (size 0.5 1.1) (layers "F.Cu" "F.Mask" "F.Paste") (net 20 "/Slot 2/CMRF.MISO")
   (solder_mask_margin 0.102))
  (pad "33" smd rect (at -3.2 -2.25) (size 0.5 1.1) (layers "F.Cu" "F.Mask" "F.Paste") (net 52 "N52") (solder_mask_margin 0.102))
  (pad "34" smd rect (at -3.2 2.25) (size 0.5 1.1) (layers "F.Cu" "F.Mask" "F.Paste") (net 4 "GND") (solder_mask_margin 0.102))
  (pad "35" smd rect (at -4 -2.25) (size 0.5 1.1) (layers "F.Cu" "F.Mask" "F.Paste") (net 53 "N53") (solder_mask_margin 0.102))
  (pad "36" smd rect (at -4 2.25) (size 0.5 1.1) (layers "F.Cu" "F.Mask" "F.Paste") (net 4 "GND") (solder_mask_margin 0.102))
  (pad "37" smd rect (at -4.8 -2.25) (size 0.5 1.1) (layers "F.Cu" "F.Mask" "F.Paste") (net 4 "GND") (solder_mask_margin 0.102))
  (pad "38" smd rect (at -4.8 2.25) (size 0.5 1.1) (layers "F.Cu" "F.Mask" "F.Paste") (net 23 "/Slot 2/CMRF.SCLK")
   (solder_mask_margin 0.102))
  (pad "39" smd rect (at -5.6 -2.25) (size 0.5 1.1) (layers "F.Cu" "F.Mask" "F.Paste") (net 4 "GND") (solder_mask_margin 0.102))
  (pad "40" smd rect (at -5.6 2.25) (size 0.5 1.1) (layers "F.Cu" "F.Mask" "F.Paste") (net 24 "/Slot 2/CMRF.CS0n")
   (solder_mask_margin 0.102))
  (pad "41" smd rect (at -6.4 -2.25) (size 0.5 1.1) (layers "F.Cu" "F.Mask" "F.Paste") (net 29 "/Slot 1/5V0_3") (solder_mask_margin 0.102))
  (pad "42" smd rect (at -6.4 2.25) (size 0.5 1.1) (layers "F.Cu" "F.Mask" "F.Paste") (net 4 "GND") (solder_mask_margin 0.102))
  (pad "43" smd rect (at -7.2 -2.25) (size 0.5 1.1) (layers "F.Cu" "F.Mask" "F.Paste") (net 29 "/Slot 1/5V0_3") (solder_mask_margin 0.102))
  (pad "44" smd rect (at -7.2 2.25) (size 0.5 1.1) (layers "F.Cu" "F.Mask" "F.Paste") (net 4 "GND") (solder_mask_margin 0.102))
  (pad "45" smd rect (at -8 -2.25) (size 0.5 1.1) (layers "F.Cu" "F.Mask" "F.Paste") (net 29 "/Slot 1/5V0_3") (solder_mask_margin 0.102))
  (pad "46" smd rect (at -8 2.25) (size 0.5 1.1) (layers "F.Cu" "F.Mask" "F.Paste") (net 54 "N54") (solder_mask_margin 0.102))
  (pad "47" smd rect (at -8.8 -2.25) (size 0.5 1.1) (layers "F.Cu" "F.Mask" "F.Paste") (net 29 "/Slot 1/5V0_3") (solder_mask_margin 0.102))
  (pad "48" smd rect (at -8.8 2.25) (size 0.5 1.1) (layers "F.Cu" "F.Mask" "F.Paste") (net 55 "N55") (solder_mask_margin 0.102))
  (pad "49" smd rect (at -9.6 -2.25) (size 0.5 1.1) (layers "F.Cu" "F.Mask" "F.Paste") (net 29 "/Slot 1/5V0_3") (solder_mask_margin 0.102))
  (pad "50" smd rect (at -9.6 2.25) (size 0.5 1.1) (layers "F.Cu" "F.Mask" "F.Paste") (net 4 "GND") (solder_mask_margin 0.102))
  (pad "S1" thru_hole circle (at -12.9 0) (size 1.338 1.338) (drill 0.83) (layers "*.Cu" "*.Mask") (remove_unused_layers no)
   (solder_mask_margin 0.102))
  (pad "S2" thru_hole circle (at 12.9 0) (size 1.338 1.338) (drill 0.83) (layers "*.Cu" "*.Mask") (remove_unused_layers no)
   (solder_mask_margin 0.102)))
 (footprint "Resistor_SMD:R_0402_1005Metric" (layer "F.Cu") (at 176.3475 95.18)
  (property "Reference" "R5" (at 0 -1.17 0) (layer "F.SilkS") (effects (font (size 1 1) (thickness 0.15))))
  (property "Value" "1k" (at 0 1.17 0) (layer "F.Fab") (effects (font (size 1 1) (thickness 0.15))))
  (pad "1" smd roundrect (at -0.51 0) (size 0.54 0.64) (layers "F.Cu" "F.Mask" "F.Paste") (roundrect_rratio 0.25) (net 28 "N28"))
  (pad "2" smd roundrect (at 0.51 0) (size 0.54 0.64) (layers "F.Cu" "F.Mask" "F.Paste") (roundrect_rratio 0.25) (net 4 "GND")))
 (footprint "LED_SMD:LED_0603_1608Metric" (layer "F.Cu") (at 172.8875 91.5)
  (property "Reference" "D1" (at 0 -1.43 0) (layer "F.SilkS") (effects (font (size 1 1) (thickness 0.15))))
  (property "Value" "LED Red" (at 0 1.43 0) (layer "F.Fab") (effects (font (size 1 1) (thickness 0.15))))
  (pad "1" smd roundrect (at -0.7875 0) (size 0.875 0.95) (layers "F.Cu" "F.Mask" "F.Paste") (roundrect_rratio 0.25) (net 31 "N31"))
  (pad "2" smd roundrect (at 0.7875 0) (size 0.875 0.95) (layers "F.Cu" "F.Mask" "F.Paste") (roundrect_rratio 0.25) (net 25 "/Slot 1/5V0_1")))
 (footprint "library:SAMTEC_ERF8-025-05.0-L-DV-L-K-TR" (layer "F.Cu") (at 153 81.525)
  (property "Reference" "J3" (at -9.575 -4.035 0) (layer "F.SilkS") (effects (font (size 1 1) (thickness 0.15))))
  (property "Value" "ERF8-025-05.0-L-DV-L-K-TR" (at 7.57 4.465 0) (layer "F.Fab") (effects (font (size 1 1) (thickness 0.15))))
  (pad "" np_thru_hole circle (at -11.4 1.5) (size 1.45 1.45) (drill 1.45) (layers "*.Cu" "*.Mask"))
  (pad "" np_thru_hole circle (at 11.4 1.5) (size 1.45 1.45) (drill 1.45) (layers "*.Cu" "*.Mask"))
  (pad "01" smd rect (at 9.6 -2.25) (size 0.5 1.1) (layers "F.Cu" "F.Mask" "F.Paste") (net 5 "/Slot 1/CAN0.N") (solder_mask_margin 0.102))
  (pad "02" smd rect (at 9.6 2.25) (size 0.5 1.1) (layers "F.Cu" "F.Mask" "F.Paste") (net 4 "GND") (solder_mask_margin 0.102))
  (pad "03" smd rect (at 8.8 -2.25) (size 0.5 1.1) (layers "F.Cu" "F.Mask" "F.Paste") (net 6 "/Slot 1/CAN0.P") (solder_mask_margin 0.102))
  (pad "04" smd rect (at 8.8 2.25) (size 0.5 1.1) (layers "F.Cu" "F.Mask" "F.Paste") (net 4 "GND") (solder_mask_margin 0.102))
  (pad "05" smd rect (at 8 -2.25) (size 0.5 1.1) (layers "F.Cu" "F.Mask" "F.Paste") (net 4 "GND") (solder_mask_margin 0.102))
  (pad "06" smd rect (at 8 2.25) (size 0.5 1.1) (layers "F.Cu" "F.Mask" "F.Paste") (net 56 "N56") (solder_mask_margin 0.102))
  (pad "07" smd rect (at 7.2 -2.25) (size 0.5 1.1) (layers "F.Cu" "F.Mask" "F.Paste") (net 4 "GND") (solder_mask_margin 0.102))
  (pad "08" smd rect (at 7.2 2.25) (size 0.5 1.1) (layers "F.Cu" "F.Mask" "F.Paste") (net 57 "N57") (solder_mask_margin 0.102))
  (pad "09" smd rect (at 6.4 -2.25) (size 0.5 1.1) (layers "F.Cu" "F.Mask" "F.Paste") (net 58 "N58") (solder_mask_margin 0.102))
  (pad "10" smd rect (at 6.4 2.25) (size 0.5 1.1) (layers "F.Cu" "F.Mask" "F.Paste") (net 4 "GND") (solder_mask_margin 0.102))
  (pad "11" smd rect (at 5.6 -2.25) (size 0.5 1.1) (layers "F.Cu" "F.Mask" "F.Paste") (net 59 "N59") (solder_mask_margin 0.102))
  (pad "12" smd rect (at 5.6 2.25) (size 0.5 1.1) (layers "F.Cu" "F.Mask" "F.Paste") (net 4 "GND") (solder_mask_margin 0.102))
  (pad "13" smd rect (at 4.8 -2.25) (size 0.5 1.1) (layers "F.Cu" "F.Mask" "F.Paste") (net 4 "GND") (solder_mask_margin 0.102))
  (pad "14" smd rect (at 4.8 2.25) (size 0.5 1.1) (layers "F.Cu" "F.Mask" "F.Paste") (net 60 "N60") (solder_mask_margin 0.102))
  (pad "15" smd rect (at 4 -2.25) (size 0.5 1.1) (layers "F.Cu" "F.Mask" "F.Paste") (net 4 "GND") (solder_mask_margin 0.102))
  (pad "16" smd rect (at 4 2.25) (size 0.5 1.1) (layers "F.Cu" "F.Mask" "F.Paste") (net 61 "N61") (solder_mask_margin 0.102))
  (pad "17" smd rect (at 3.2 -2.25) (size 0.5 1.1) (layers "F.Cu" "F.Mask" "F.Paste") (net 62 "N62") (solder_mask_margin 0.102))
  (pad "18" smd rect (at 3.2 2.25) (size 0.5 1.1) (layers "F.Cu" "F.Mask" "F.Paste") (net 4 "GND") (solder_mask_margin 0.102))
  (pad "19" smd rect (at 2.4 -2.25) (size 0.5 1.1) (layers "F.Cu" "F.Mask" "F.Paste") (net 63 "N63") (solder_mask_margin 0.102))
  (pad "20" smd rect (at 2.4 2.25) (size 0.5 1.1) (layers "F.Cu" "F.Mask" "F.Paste") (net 4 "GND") (solder_mask_margin 0.102))
  (pad "21" smd rect (at 1.6 -2.25) (size 0.5 1.1) (layers "F.Cu" "F.Mask" "F.Paste") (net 4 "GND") (solder_mask_margin 0.102))
  (pad "22" smd rect (at 1.6 2.25) (size 0.5 1.1) (layers "F.Cu" "F.Mask" "F.Paste") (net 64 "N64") (solder_mask_margin 0.102))
  (pad "23" smd rect (at 0.8 -2.25) (size 0.5 1.1) (layers "F.Cu" "F.Mask" "F.Paste") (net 4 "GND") (solder_mask_margin 0.102))
  (pad "24" smd rect (at 0.8 2.25) (size 0.5 1.1) (layers "F.Cu" "F.Mask" "F.Paste") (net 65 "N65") (solder_mask_margin 0.102))
  (pad "25" smd rect (at 0 -2.25) (size 0.5 1.1) (layers "F.Cu" "F.Mask" "F.Paste") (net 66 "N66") (solder_mask_margin 0.102))
  (pad "26" smd rect (at 0 2.25) (size 0.5 1.1) (layers "F.Cu" "F.Mask" "F.Paste") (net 4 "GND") (solder_mask_margin 0.102))
  (pad "27" smd rect (at -0.8 -2.25) (size 0.5 1.1) (layers "F.Cu" "F.Mask" "F.Paste") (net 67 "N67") (solder_mask_margin 0.102))
  (pad "28" smd rect (at -0.8 2.25) (size 0.5 1.1) (layers "F.Cu" "F.Mask" "F.Paste") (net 4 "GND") (solder_mask_margin 0.102))
  (pad "29" smd rect (at -1.6 -2.25) (size 0.5 1.1) (layers "F.Cu" "F.Mask" "F.Paste") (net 4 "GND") (solder_mask_margin 0.102))
  (pad "30" smd rect (at -1.6 2.25) (size 0.5 1.1) (layers "F.Cu" "F.Mask" "F.Paste") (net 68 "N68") (solder_mask_margin 0.102))
  (pad "31" smd rect (at -2.4 -2.25) (size 0.5 1.1) (layers "F.Cu" "F.Mask" "F.Paste") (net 4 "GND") (solder_mask_margin 0.102))
  (pad "32" smd rect (at -2.4 2.25) (size 0.5 1.1) (layers "F.Cu" "F.Mask" "F.Paste") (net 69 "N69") (solder_mask_margin 0.102))
  (pad "33" smd rect (at -3.2 -2.25) (size 0.5 1.1) (layers "F.Cu" "F.Mask" "F.Paste") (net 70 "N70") (solder_mask_margin 0.102))
  (pad "34" smd rect (at -3.2 2.25) (size 0.5 1.1) (layers "F.Cu" "F.Mask" "F.Paste") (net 4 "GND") (solder_mask_margin 0.102))
  (pad "35" smd rect (at -4 -2.25) (size 0.5 1.1) (layers "F.Cu" "F.Mask" "F.Paste") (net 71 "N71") (solder_mask_margin 0.102))
  (pad "36" smd rect (at -4 2.25) (size 0.5 1.1) (layers "F.Cu" "F.Mask" "F.Paste") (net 4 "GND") (solder_mask_margin 0.102))
  (pad "37" smd rect (at -4.8 -2.25) (size 0.5 1.1) (layers "F.Cu" "F.Mask" "F.Paste") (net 4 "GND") (solder_mask_margin 0.102))
  (pad "38" smd rect (at -4.8 2.25) (size 0.5 1.1) (layers "F.Cu" "F.Mask" "F.Paste") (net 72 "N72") (solder_mask_margin 0.102))
  (pad "39" smd rect (at -5.6 -2.25) (size 0.5 1.1) (layers "F.Cu" "F.Mask" "F.Paste") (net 4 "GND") (solder_mask_margin 0.102))
  (pad "40" smd rect (at -5.6 2.25) (size 0.5 1.1) (layers "F.Cu" "F.Mask" "F.Paste") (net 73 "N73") (solder_mask_margin 0.102))
  (pad "41" smd rect (at -6.4 -2.25) (size 0.5 1.1) (layers "F.Cu" "F.Mask" "F.Paste") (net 2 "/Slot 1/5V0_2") (solder_mask_margin 0.102))
  (pad "42" smd rect (at -6.4 2.25) (size 0.5 1.1) (layers "F.Cu" "F.Mask" "F.Paste") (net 4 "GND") (solder_mask_margin 0.102))
  (pad "43" smd rect (at -7.2 -2.25) (size 0.5 1.1) (layers "F.Cu" "F.Mask" "F.Paste") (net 2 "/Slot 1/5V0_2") (solder_mask_margin 0.102))
  (pad "44" smd rect (at -7.2 2.25) (size 0.5 1.1) (layers "F.Cu" "F.Mask" "F.Paste") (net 4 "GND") (solder_mask_margin 0.102))
  (pad "45" smd rect (at -8 -2.25) (size 0.5 1.1) (layers "F.Cu" "F.Mask" "F.Paste") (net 2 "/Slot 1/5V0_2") (solder_mask_margin 0.102))
  (pad "46" smd rect (at -8 2.25) (size 0.5 1.1) (layers "F.Cu" "F.Mask" "F.Paste") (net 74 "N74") (solder_mask_margin 0.102))
  (pad "47" smd rect (at -8.8 -2.25) (size 0.5 1.1) (layers "F.Cu" "F.Mask" "F.Paste") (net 2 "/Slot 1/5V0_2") (solder_mask_margin 0.102))
  (pad "48" smd rect (at -8.8 2.25) (size 0.5 1.1) (layers "F.Cu" "F.Mask" "F.Paste") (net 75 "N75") (solder_mask_margin 0.102))
  (pad "49" smd rect (at -9.6 -2.25) (size 0.5 1.1) (layers "F.Cu" "F.Mask" "F.Paste") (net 2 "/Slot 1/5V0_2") (solder_mask_margin 0.102))
  (pad "50" smd rect (at -9.6 2.25) (size 0.5 1.1) (layers "F.Cu" "F.Mask" "F.Paste") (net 4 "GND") (solder_mask_margin 0.102))
  (pad "S1" thru_hole circle (at -12.9 0) (size 1.338 1.338) (drill 0.83) (layers "*.Cu" "*.Mask") (remove_unused_layers no)
   (solder_mask_margin 0.102))
  (pad "S2" thru_hole circle (at 12.9 0) (size 1.338 1.338) (drill 0.83) (layers "*.Cu" "*.Mask") (remove_unused_layers no)
   (solder_mask_margin 0.102)))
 (gr_circle (center 178.5 52) (end 178.5 53.675) (stroke (width 0.25) (type default)) (fill no) (layer "Edge.Cuts"))
 (gr_line (start 126.25 135) (end 179.75 135) (stroke (width 0.25) (type default)) (layer "Edge.Cuts"))
 (gr_arc (start 124.25 50.999998) (mid 124.835786 49.585786) (end 126.249998 49) (stroke (width 0.25) (type default)) (layer "Edge.Cuts"))
 (gr_line (start 181.75 133) (end 181.75 50.999998) (stroke (width 0.25) (type default)) (layer "Edge.Cuts"))
 (gr_circle (center 127.5 52) (end 127.5 53.675) (stroke (width 0.25) (type default)) (fill no) (layer "Edge.Cuts"))
 (gr_circle (center 178.5 117) (end 178.5 118.675) (stroke (width 0.25) (type default)) (fill no) (layer "Edge.Cuts"))
 (gr_line (start 124.25 50.999998) (end 124.25 133) (stroke (width 0.25) (type default)) (layer "Edge.Cuts"))
 (gr_line (start 179.750001 49) (end 126.249998 49) (stroke (width 0.25) (type default)) (layer "Edge.Cuts"))
 (gr_arc (start 181.75 133) (mid 181.164214 134.414214) (end 179.75 135) (stroke (width 0.25) (type default)) (layer "Edge.Cuts"))
 (gr_arc (start 126.25 135) (mid 124.835786 134.414214) (end 124.25 133) (stroke (width 0.25) (type default)) (layer "Edge.Cuts"))
 (gr_circle (center 127.5 117) (end 127.5 118.675) (stroke (width 0.25) (type default)) (fill no) (layer "Edge.Cuts"))
 (gr_arc (start 179.750001 49) (mid 181.164214 49.585786) (end 181.75 50.999998) (stroke (width 0.25) (type default)) (layer "Edge.Cuts"))
 (segment (start 161.8 53.729999) (end 161.975 53.554999) (width 0.2) (layer "F.Cu") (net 6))
 (segment (start 161.975 127.714999) (end 161.975 127.112501) (width 0.2) (layer "F.Cu") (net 6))
 (segment (start 161.975 127.112501) (end 161.375 126.512501) (width 0.2) (layer "F.Cu") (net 6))
 (segment (start 161.8 127.889999) (end 161.975 127.714999) (width 0.2) (layer "F.Cu") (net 6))
 (segment (start 161.375 52.112501) (end 161.375 51.4) (width 0.2) (layer "F.Cu") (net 6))
 (segment (start 161.375 126.512501) (end 161.375 125.8) (width 0.2) (layer "F.Cu") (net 6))
 (segment (start 161.8 54.555) (end 161.8 53.729999) (width 0.2) (layer "F.Cu") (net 6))
 (segment (start 161.975 53.554999) (end 161.975 52.712501) (width 0.2) (layer "F.Cu") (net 6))
 (segment (start 161.975 52.712501) (end 161.375 52.112501) (width 0.2) (layer "F.Cu") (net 6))
 (segment (start 161.8 128.715) (end 161.8 127.889999) (width 0.2) (layer "F.Cu") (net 6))
 (segment (start 162.6 54.555) (end 162.6 53.729999) (width 0.2) (layer "F.Cu") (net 5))
 (segment (start 163.025 126.512501) (end 163.025 125.8) (width 0.2) (layer "F.Cu") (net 5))
 (segment (start 163.025 52.112501) (end 163.025 51.4) (width 0.2) (layer "F.Cu") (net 5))
 (segment (start 162.6 128.715) (end 162.6 127.889999) (width 0.2) (layer "F.Cu") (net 5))
 (segment (start 162.6 127.889999) (end 162.425 127.714999) (width 0.2) (layer "F.Cu") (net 5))
 (segment (start 162.425 53.554999) (end 162.425 52.712501) (width 0.2) (layer "F.Cu") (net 5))
 (segment (start 162.425 127.112501) (end 163.025 126.512501) (width 0.2) (layer "F.Cu") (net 5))
 (segment (start 162.6 53.729999) (end 162.425 53.554999) (width 0.2) (layer "F.Cu") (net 5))
 (segment (start 162.425 127.714999) (end 162.425 127.112501) (width 0.2) (layer "F.Cu") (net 5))
 (segment (start 162.425 52.712501) (end 163.025 52.112501) (width 0.2) (layer "F.Cu") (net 5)))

